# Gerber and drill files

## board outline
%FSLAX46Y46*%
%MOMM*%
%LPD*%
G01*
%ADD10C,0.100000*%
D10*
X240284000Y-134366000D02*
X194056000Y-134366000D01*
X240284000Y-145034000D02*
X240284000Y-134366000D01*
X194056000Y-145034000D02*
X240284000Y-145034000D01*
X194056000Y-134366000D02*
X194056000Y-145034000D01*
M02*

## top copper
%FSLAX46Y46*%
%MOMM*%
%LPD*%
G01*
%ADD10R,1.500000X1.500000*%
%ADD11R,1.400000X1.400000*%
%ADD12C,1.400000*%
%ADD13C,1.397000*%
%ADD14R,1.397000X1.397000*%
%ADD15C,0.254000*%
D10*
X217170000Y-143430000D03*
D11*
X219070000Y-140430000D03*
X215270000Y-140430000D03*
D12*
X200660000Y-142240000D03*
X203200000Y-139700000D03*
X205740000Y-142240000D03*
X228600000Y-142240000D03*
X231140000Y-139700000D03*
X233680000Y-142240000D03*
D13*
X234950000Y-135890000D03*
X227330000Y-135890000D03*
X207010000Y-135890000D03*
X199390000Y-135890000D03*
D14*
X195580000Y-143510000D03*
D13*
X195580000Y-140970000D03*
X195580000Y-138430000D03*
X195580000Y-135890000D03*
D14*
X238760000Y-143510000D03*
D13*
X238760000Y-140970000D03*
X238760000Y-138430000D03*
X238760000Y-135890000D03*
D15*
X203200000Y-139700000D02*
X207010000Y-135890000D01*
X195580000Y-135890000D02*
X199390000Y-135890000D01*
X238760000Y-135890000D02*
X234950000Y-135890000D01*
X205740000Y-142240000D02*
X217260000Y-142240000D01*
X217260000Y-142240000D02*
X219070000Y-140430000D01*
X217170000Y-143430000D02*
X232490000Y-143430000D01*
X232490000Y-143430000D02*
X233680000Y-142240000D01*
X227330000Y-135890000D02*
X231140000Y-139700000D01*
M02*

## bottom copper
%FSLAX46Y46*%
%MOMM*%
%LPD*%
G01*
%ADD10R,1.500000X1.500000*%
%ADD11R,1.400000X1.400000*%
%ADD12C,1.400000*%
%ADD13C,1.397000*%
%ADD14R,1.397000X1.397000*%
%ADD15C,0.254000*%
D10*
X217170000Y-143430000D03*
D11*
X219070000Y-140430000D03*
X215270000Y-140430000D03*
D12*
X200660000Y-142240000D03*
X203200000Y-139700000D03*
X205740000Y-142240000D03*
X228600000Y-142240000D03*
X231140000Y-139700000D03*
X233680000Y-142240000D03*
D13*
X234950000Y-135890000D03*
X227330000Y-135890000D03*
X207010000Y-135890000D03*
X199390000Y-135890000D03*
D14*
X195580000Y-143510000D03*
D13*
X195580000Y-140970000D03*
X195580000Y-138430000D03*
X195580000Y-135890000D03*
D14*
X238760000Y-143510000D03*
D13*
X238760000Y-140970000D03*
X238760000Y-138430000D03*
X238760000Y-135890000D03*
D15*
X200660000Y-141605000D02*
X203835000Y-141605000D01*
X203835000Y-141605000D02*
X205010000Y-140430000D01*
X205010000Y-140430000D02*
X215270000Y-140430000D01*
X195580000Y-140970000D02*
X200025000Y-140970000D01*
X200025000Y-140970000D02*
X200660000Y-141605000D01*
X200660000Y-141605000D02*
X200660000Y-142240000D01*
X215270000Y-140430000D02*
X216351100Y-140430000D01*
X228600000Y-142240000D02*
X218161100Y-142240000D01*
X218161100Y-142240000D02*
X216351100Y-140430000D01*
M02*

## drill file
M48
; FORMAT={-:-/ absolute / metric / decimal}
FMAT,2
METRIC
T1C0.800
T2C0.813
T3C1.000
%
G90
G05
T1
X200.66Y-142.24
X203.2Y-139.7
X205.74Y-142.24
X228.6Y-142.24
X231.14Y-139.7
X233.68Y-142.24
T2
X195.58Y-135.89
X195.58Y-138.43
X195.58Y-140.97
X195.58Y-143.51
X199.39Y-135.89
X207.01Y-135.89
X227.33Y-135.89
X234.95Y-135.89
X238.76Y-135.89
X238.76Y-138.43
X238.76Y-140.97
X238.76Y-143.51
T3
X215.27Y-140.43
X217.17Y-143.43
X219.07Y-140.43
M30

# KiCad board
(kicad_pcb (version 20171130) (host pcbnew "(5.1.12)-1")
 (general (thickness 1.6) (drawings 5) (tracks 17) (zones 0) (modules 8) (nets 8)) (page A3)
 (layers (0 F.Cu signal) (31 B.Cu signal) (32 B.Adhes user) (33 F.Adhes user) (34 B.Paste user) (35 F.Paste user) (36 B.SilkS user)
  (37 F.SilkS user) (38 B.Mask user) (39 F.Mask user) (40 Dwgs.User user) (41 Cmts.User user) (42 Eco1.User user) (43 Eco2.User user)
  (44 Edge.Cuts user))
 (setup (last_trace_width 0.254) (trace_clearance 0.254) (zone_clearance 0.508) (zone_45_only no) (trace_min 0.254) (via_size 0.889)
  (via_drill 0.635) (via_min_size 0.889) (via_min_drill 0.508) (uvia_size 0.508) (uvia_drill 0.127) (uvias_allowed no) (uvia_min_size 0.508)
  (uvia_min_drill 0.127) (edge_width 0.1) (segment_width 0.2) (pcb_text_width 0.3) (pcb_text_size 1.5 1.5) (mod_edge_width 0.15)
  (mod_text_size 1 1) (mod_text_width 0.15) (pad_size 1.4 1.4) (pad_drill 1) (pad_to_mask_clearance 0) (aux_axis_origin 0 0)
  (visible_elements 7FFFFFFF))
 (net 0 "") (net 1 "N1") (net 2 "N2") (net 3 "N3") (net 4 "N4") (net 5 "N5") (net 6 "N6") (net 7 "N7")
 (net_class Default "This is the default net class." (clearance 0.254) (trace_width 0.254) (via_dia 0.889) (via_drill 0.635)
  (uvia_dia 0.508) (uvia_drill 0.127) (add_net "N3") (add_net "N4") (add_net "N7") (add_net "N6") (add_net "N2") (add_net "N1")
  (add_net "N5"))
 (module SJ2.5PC (layer F.Cu) (at 217.17 138.43 270)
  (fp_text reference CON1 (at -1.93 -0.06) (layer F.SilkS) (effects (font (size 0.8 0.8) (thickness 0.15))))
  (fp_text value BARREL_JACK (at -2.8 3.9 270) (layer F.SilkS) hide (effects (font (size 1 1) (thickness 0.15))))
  (pad 3 thru_hole rect (at 5 0 270) (size 1.5 1.5) (drill 1) (layers *.Cu *.Mask F.SilkS) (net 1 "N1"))
  (pad 2 thru_hole rect (at 2 -1.9 270) (size 1.4 1.4) (drill 1) (layers *.Cu *.Mask F.SilkS) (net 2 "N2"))
  (pad 1 thru_hole rect (at 2 1.9 270) (size 1.4 1.4) (drill 1) (layers *.Cu *.Mask F.SilkS) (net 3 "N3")))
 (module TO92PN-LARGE (layer F.Cu) (at 203.2 139.7 180)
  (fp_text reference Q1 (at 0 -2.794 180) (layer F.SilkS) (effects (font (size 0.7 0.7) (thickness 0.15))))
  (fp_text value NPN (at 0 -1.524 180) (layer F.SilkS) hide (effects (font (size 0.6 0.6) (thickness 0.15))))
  (pad 1 thru_hole circle (at 2.54 -2.54 180) (size 1.4 1.4) (drill 0.8) (layers *.Cu *.Mask F.SilkS) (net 3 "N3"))
  (pad 2 thru_hole circle (at 0 0 180) (size 1.4 1.4) (drill 0.8) (layers *.Cu *.Mask F.SilkS) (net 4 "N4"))
  (pad 3 thru_hole circle (at -2.54 -2.54 180) (size 1.4 1.4) (drill 0.8) (layers *.Cu *.Mask F.SilkS) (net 2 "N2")))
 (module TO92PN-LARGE (layer F.Cu) (at 231.14 139.7 180)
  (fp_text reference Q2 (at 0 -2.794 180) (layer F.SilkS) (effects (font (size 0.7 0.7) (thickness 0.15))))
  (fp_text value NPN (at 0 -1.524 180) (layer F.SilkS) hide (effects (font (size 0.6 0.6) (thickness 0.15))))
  (pad 1 thru_hole circle (at 2.54 -2.54 180) (size 1.4 1.4) (drill 0.8) (layers *.Cu *.Mask F.SilkS) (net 3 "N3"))
  (pad 2 thru_hole circle (at 0 0 180) (size 1.4 1.4) (drill 0.8) (layers *.Cu *.Mask F.SilkS) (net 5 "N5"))
  (pad 3 thru_hole circle (at -2.54 -2.54 180) (size 1.4 1.4) (drill 0.8) (layers *.Cu *.Mask F.SilkS) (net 1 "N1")))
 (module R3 (layer F.Cu) (at 231.14 135.89 180) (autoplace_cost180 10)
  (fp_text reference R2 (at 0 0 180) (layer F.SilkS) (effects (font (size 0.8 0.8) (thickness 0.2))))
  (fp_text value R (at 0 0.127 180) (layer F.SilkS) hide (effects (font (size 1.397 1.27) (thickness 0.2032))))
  (pad 1 thru_hole circle (at -3.81 0 180) (size 1.397 1.397) (drill 0.8128) (layers *.Cu *.Mask F.SilkS) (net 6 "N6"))
  (pad 2 thru_hole circle (at 3.81 0 180) (size 1.397 1.397) (drill 0.8128) (layers *.Cu *.Mask F.SilkS) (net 5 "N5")))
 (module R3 (layer F.Cu) (at 203.2 135.89 180) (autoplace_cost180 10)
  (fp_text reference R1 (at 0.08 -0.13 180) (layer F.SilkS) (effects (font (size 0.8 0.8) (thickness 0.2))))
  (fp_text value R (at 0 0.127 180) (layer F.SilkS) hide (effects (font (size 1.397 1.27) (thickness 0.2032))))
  (pad 1 thru_hole circle (at -3.81 0 180) (size 1.397 1.397) (drill 0.8128) (layers *.Cu *.Mask F.SilkS) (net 4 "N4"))
  (pad 2 thru_hole circle (at 3.81 0 180) (size 1.397 1.397) (drill 0.8128) (layers *.Cu *.Mask F.SilkS) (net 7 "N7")))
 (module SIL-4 (layer F.Cu) (at 195.58 139.7 90)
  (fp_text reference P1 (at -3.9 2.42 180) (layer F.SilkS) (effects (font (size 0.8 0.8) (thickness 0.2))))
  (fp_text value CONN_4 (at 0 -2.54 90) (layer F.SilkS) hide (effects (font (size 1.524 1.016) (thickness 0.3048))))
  (pad 1 thru_hole rect (at -3.81 0 90) (size 1.397 1.397) (drill 0.8128) (layers *.Cu *.Mask F.SilkS))
  (pad 2 thru_hole circle (at -1.27 0 90) (size 1.397 1.397) (drill 0.8128) (layers *.Cu *.Mask F.SilkS) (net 3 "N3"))
  (pad 3 thru_hole circle (at 1.27 0 90) (size 1.397 1.397) (drill 0.8128) (layers *.Cu *.Mask F.SilkS))
  (pad 4 thru_hole circle (at 3.81 0 90) (size 1.397 1.397) (drill 0.8128) (layers *.Cu *.Mask F.SilkS) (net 7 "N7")))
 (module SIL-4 (layer F.Cu) (at 238.76 139.7 90)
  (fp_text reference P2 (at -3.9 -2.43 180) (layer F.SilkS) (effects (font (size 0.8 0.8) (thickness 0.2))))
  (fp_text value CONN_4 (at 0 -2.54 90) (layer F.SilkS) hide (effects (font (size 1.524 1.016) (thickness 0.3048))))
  (pad 1 thru_hole rect (at -3.81 0 90) (size 1.397 1.397) (drill 0.8128) (layers *.Cu *.Mask F.SilkS))
  (pad 2 thru_hole circle (at -1.27 0 90) (size 1.397 1.397) (drill 0.8128) (layers *.Cu *.Mask F.SilkS))
  (pad 3 thru_hole circle (at 1.27 0 90) (size 1.397 1.397) (drill 0.8128) (layers *.Cu *.Mask F.SilkS))
  (pad 4 thru_hole circle (at 3.81 0 90) (size 1.397 1.397) (drill 0.8128) (layers *.Cu *.Mask F.SilkS) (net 6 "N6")))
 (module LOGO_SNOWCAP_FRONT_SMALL (layer F.Cu) (at 210.82 139.446 90)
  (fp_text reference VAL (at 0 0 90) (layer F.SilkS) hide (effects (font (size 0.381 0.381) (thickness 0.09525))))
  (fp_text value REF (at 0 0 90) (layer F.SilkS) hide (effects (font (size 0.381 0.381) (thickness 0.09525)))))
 (gr_line (start 240.284 134.366) (end 194.056 134.366) (angle 90) (layer Edge.Cuts) (width 0.1))
 (gr_line (start 240.284 145.034) (end 240.284 134.366) (angle 90) (layer Edge.Cuts) (width 0.1))
 (gr_line (start 194.056 145.034) (end 240.284 145.034) (angle 90) (layer Edge.Cuts) (width 0.1))
 (gr_line (start 194.056 134.366) (end 194.056 145.034) (angle 90) (layer Edge.Cuts) (width 0.1))
 (segment (start 200.66 141.605) (end 203.835 141.605) (width 0.254) (layer B.Cu) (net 3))
 (segment (start 203.835 141.605) (end 205.01 140.43) (width 0.254) (layer B.Cu) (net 3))
 (segment (start 205.01 140.43) (end 215.27 140.43) (width 0.254) (layer B.Cu) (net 3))
 (segment (start 195.58 140.97) (end 200.025 140.97) (width 0.254) (layer B.Cu) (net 3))
 (segment (start 200.025 140.97) (end 200.66 141.605) (width 0.254) (layer B.Cu) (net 3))
 (segment (start 200.66 141.605) (end 200.66 142.24) (width 0.254) (layer B.Cu) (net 3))
 (segment (start 215.27 140.43) (end 216.3511 140.43) (width 0.254) (layer B.Cu) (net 3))
 (segment (start 228.6 142.24) (end 218.1611 142.24) (width 0.254) (layer B.Cu) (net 3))
 (segment (start 218.1611 142.24) (end 216.3511 140.43) (width 0.254) (layer B.Cu) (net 3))
 (segment (start 203.2 139.7) (end 207.01 135.89) (width 0.254) (layer F.Cu) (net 4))
 (segment (start 195.58 135.89) (end 199.39 135.89) (width 0.254) (layer F.Cu) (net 7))
 (segment (start 238.76 135.89) (end 234.95 135.89) (width 0.254) (layer F.Cu) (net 6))
 (segment (start 205.74 142.24) (end 217.26 142.24) (width 0.254) (layer F.Cu) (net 2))
 (segment (start 217.26 142.24) (end 219.07 140.43) (width 0.254) (layer F.Cu) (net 2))
 (segment (start 217.17 143.43) (end 232.49 143.43) (width 0.254) (layer F.Cu) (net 1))
 (segment (start 232.49 143.43) (end 233.68 142.24) (width 0.254) (layer F.Cu) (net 1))
 (segment (start 227.33 135.89) (end 231.14 139.7) (width 0.254) (layer F.Cu) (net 5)))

